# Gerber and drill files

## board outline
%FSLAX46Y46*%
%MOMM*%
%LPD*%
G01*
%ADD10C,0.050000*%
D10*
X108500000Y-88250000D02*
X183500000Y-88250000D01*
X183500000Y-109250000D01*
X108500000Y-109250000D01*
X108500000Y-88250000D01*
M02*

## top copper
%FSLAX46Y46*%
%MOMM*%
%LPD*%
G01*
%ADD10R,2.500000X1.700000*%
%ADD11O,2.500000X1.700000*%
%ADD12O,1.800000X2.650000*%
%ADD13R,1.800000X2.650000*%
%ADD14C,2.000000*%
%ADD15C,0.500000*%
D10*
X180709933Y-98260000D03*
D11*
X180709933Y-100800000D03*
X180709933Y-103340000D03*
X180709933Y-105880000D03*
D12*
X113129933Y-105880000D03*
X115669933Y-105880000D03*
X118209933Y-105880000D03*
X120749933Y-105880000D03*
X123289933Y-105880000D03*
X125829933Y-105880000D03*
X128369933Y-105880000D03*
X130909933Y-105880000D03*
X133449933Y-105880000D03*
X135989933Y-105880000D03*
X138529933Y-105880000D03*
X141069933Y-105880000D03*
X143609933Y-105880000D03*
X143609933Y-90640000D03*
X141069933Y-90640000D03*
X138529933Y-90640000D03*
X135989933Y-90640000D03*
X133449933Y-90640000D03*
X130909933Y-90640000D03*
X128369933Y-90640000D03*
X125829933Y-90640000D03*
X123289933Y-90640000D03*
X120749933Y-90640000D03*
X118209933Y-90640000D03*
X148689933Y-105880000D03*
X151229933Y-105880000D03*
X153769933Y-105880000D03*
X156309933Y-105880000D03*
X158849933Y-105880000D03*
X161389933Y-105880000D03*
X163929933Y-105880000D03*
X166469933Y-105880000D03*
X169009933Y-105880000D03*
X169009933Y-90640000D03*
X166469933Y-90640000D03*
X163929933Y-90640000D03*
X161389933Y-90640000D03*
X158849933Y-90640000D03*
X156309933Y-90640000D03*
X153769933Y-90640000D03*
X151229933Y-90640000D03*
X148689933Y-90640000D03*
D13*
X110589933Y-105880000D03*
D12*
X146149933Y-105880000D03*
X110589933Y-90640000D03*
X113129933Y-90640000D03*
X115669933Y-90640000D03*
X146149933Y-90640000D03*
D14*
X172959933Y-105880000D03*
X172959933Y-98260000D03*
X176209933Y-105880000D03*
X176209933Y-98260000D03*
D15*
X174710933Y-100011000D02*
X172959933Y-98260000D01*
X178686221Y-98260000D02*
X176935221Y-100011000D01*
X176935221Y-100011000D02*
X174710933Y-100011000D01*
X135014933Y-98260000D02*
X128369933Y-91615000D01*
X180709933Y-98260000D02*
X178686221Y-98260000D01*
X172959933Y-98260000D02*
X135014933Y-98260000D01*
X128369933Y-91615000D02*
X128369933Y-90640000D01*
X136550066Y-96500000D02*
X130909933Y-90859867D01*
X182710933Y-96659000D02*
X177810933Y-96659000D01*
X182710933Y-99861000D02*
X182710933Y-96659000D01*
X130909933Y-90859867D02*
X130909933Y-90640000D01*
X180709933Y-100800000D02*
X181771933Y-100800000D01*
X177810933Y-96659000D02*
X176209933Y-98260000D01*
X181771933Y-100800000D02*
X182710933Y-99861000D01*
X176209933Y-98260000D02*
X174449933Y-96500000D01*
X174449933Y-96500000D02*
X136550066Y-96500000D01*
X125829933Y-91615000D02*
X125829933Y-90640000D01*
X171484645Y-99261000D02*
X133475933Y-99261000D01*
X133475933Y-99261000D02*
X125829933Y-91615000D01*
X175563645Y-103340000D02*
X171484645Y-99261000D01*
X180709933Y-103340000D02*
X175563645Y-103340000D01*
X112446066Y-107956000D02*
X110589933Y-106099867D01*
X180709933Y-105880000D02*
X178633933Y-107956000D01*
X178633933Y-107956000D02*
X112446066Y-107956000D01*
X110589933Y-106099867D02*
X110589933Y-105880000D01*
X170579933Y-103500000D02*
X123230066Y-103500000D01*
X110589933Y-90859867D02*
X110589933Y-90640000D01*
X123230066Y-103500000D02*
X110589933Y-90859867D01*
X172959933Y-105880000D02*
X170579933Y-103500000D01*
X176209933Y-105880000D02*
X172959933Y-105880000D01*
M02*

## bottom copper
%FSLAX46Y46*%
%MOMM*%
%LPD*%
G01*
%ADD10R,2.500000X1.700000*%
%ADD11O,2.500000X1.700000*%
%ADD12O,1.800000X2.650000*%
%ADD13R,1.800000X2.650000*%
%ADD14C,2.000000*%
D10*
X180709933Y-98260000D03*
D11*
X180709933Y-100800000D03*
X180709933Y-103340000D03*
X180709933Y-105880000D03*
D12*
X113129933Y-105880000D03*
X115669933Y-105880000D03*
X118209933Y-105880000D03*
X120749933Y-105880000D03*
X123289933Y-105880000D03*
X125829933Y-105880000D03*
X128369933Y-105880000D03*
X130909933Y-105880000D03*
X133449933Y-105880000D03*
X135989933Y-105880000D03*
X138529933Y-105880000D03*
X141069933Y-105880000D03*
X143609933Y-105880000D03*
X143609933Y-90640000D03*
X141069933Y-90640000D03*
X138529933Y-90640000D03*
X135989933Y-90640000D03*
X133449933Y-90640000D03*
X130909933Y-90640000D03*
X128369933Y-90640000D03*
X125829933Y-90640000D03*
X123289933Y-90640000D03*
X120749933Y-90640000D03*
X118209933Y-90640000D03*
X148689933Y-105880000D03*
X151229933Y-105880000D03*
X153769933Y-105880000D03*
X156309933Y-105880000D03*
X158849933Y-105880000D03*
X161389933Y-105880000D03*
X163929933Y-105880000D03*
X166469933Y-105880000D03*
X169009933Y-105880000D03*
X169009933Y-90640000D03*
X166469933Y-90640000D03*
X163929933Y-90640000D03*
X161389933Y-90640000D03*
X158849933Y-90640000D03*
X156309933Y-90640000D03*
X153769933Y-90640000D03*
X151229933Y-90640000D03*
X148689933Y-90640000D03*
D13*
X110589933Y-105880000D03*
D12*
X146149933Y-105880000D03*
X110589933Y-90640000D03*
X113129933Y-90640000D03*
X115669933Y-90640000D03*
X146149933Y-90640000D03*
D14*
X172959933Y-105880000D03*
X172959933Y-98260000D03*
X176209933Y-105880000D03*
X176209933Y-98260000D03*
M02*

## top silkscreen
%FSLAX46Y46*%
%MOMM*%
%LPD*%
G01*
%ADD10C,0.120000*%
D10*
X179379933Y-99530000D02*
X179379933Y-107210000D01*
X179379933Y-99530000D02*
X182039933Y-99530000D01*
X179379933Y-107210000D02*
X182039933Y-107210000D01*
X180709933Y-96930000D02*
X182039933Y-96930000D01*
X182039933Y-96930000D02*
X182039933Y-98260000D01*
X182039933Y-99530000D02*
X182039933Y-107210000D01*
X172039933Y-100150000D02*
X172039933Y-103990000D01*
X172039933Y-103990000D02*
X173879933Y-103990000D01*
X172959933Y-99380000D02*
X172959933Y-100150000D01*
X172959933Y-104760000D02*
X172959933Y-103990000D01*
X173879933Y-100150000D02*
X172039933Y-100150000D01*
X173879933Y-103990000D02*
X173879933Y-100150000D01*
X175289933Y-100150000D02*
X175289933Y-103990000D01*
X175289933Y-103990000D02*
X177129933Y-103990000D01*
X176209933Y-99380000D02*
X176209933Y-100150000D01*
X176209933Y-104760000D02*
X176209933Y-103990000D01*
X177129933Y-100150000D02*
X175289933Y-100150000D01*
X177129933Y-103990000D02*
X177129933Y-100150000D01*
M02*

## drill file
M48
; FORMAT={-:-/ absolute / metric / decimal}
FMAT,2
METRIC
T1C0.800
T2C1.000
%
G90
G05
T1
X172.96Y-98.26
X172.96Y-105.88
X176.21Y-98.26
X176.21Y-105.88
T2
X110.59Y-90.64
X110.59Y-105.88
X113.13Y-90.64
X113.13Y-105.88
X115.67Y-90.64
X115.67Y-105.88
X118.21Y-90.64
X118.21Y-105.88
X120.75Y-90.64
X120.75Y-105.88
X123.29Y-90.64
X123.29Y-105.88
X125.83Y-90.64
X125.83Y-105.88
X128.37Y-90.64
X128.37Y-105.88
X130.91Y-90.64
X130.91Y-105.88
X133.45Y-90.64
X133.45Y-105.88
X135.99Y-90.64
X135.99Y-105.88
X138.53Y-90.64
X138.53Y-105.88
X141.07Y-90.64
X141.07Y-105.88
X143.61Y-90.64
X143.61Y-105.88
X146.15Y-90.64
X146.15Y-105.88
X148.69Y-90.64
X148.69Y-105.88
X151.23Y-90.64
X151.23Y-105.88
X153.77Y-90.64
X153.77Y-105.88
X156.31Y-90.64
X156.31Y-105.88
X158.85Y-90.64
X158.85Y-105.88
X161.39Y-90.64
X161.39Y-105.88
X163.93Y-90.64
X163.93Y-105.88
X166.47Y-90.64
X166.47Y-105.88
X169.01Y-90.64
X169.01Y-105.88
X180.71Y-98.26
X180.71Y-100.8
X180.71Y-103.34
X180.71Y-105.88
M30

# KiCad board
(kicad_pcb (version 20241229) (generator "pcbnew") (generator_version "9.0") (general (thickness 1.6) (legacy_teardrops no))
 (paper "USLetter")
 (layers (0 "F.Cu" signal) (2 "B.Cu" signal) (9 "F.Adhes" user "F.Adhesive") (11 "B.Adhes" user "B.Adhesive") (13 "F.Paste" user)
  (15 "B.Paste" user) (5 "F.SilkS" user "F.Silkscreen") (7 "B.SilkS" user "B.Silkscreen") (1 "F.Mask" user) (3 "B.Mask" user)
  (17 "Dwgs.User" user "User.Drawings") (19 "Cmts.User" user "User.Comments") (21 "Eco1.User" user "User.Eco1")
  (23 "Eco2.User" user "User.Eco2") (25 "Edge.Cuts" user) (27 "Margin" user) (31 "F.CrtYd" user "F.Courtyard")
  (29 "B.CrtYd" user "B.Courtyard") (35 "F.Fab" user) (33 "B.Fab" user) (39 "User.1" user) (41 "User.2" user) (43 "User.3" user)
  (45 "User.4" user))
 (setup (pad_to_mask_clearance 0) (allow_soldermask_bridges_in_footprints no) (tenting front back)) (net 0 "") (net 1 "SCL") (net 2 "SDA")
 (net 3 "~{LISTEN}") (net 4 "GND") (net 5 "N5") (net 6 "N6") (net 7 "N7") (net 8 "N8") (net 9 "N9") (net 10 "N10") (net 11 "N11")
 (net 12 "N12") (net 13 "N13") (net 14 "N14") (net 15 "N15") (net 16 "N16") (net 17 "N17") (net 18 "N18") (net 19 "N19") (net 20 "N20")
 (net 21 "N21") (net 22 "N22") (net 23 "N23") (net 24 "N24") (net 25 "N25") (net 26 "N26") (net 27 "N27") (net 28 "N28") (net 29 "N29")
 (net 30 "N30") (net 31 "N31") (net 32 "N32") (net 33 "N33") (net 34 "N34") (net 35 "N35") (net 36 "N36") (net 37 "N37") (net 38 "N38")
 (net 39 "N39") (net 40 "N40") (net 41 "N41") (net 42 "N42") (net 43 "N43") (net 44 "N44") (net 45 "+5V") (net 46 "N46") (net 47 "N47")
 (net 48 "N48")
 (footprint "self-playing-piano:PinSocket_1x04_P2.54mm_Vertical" (layer "F.Cu") (at 180.709933 98.26)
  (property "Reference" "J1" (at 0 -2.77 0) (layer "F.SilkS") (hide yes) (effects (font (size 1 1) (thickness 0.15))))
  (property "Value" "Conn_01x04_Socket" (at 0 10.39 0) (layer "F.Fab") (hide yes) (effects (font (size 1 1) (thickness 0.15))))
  (fp_line (start -1.33 1.27) (end -1.33 8.95) (stroke (width 0.12) (type solid)) (layer "F.SilkS"))
  (fp_line (start -1.33 1.27) (end 1.33 1.27) (stroke (width 0.12) (type solid)) (layer "F.SilkS"))
  (fp_line (start -1.33 8.95) (end 1.33 8.95) (stroke (width 0.12) (type solid)) (layer "F.SilkS"))
  (fp_line (start 0 -1.33) (end 1.33 -1.33) (stroke (width 0.12) (type solid)) (layer "F.SilkS"))
  (fp_line (start 1.33 -1.33) (end 1.33 0) (stroke (width 0.12) (type solid)) (layer "F.SilkS"))
  (fp_line (start 1.33 1.27) (end 1.33 8.95) (stroke (width 0.12) (type solid)) (layer "F.SilkS"))
  (pad "1" thru_hole rect (at 0 0) (size 2.5 1.7) (drill 1) (layers "*.Cu" "*.Mask") (remove_unused_layers no) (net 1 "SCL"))
  (pad "2" thru_hole oval (at 0 2.54) (size 2.5 1.7) (drill 1) (layers "*.Cu" "*.Mask") (remove_unused_layers no) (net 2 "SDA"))
  (pad "3" thru_hole oval (at 0 5.08) (size 2.5 1.7) (drill 1) (layers "*.Cu" "*.Mask") (remove_unused_layers no) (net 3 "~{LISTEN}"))
  (pad "4" thru_hole oval (at 0 7.62) (size 2.5 1.7) (drill 1) (layers "*.Cu" "*.Mask") (remove_unused_layers no) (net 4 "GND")))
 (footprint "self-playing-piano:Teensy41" (layer "F.Cu") (at 110.589933 105.88 90)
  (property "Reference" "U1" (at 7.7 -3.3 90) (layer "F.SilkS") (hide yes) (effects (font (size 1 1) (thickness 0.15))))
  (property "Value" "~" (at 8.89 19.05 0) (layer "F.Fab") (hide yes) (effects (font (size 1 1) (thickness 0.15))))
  (pad "0" thru_hole oval (at 0 2.54 90) (size 2.65 1.8) (drill 1) (layers "*.Cu" "*.Mask") (remove_unused_layers no) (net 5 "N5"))
  (pad "1" thru_hole oval (at 0 5.08 90) (size 2.65 1.8) (drill 1) (layers "*.Cu" "*.Mask") (remove_unused_layers no) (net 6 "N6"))
  (pad "2" thru_hole oval (at 0 7.62 90) (size 2.65 1.8) (drill 1) (layers "*.Cu" "*.Mask") (remove_unused_layers no) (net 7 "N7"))
  (pad "3" thru_hole oval (at 0 10.16 90) (size 2.65 1.8) (drill 1) (layers "*.Cu" "*.Mask") (remove_unused_layers no) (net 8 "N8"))
  (pad "4" thru_hole oval (at 0 12.7 90) (size 2.65 1.8) (drill 1) (layers "*.Cu" "*.Mask") (remove_unused_layers no) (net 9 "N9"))
  (pad "5" thru_hole oval (at 0 15.24 90) (size 2.65 1.8) (drill 1) (layers "*.Cu" "*.Mask") (remove_unused_layers no) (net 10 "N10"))
  (pad "6" thru_hole oval (at 0 17.78 90) (size 2.65 1.8) (drill 1) (layers "*.Cu" "*.Mask") (remove_unused_layers no) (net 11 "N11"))
  (pad "7" thru_hole oval (at 0 20.32 90) (size 2.65 1.8) (drill 1) (layers "*.Cu" "*.Mask") (remove_unused_layers no) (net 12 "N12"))
  (pad "8" thru_hole oval (at 0 22.86 90) (size 2.65 1.8) (drill 1) (layers "*.Cu" "*.Mask") (remove_unused_layers no) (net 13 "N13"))
  (pad "9" thru_hole oval (at 0 25.4 90) (size 2.65 1.8) (drill 1) (layers "*.Cu" "*.Mask") (remove_unused_layers no) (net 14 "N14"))
  (pad "10" thru_hole oval (at 0 27.94 90) (size 2.65 1.8) (drill 1) (layers "*.Cu" "*.Mask") (remove_unused_layers no) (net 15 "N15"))
  (pad "11" thru_hole oval (at 0 30.48 90) (size 2.65 1.8) (drill 1) (layers "*.Cu" "*.Mask") (remove_unused_layers no) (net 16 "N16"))
  (pad "12" thru_hole oval (at 0 33.02 90) (size 2.65 1.8) (drill 1) (layers "*.Cu" "*.Mask") (remove_unused_layers no) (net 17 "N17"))
  (pad "13" thru_hole oval (at 15.24 33.02 90) (size 2.65 1.8) (drill 1) (layers "*.Cu" "*.Mask") (remove_unused_layers no) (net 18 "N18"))
  (pad "14" thru_hole oval (at 15.24 30.48 90) (size 2.65 1.8) (drill 1) (layers "*.Cu" "*.Mask") (remove_unused_layers no) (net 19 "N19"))
  (pad "15" thru_hole oval (at 15.24 27.94 90) (size 2.65 1.8) (drill 1) (layers "*.Cu" "*.Mask") (remove_unused_layers no) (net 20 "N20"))
  (pad "16" thru_hole oval (at 15.24 25.4 90) (size 2.65 1.8) (drill 1) (layers "*.Cu" "*.Mask") (remove_unused_layers no) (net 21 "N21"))
  (pad "17" thru_hole oval (at 15.24 22.86 90) (size 2.65 1.8) (drill 1) (layers "*.Cu" "*.Mask") (remove_unused_layers no) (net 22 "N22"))
  (pad "18" thru_hole oval (at 15.24 20.32 90) (size 2.65 1.8) (drill 1) (layers "*.Cu" "*.Mask") (remove_unused_layers no) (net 2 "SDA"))
  (pad "19" thru_hole oval (at 15.24 17.78 90) (size 2.65 1.8) (drill 1) (layers "*.Cu" "*.Mask") (remove_unused_layers no) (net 1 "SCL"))
  (pad "20" thru_hole oval (at 15.24 15.24 90) (size 2.65 1.8) (drill 1) (layers "*.Cu" "*.Mask") (remove_unused_layers no)
   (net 3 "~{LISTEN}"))
  (pad "21" thru_hole oval (at 15.24 12.7 90) (size 2.65 1.8) (drill 1) (layers "*.Cu" "*.Mask") (remove_unused_layers no) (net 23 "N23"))
  (pad "22" thru_hole oval (at 15.24 10.16 90) (size 2.65 1.8) (drill 1) (layers "*.Cu" "*.Mask") (remove_unused_layers no) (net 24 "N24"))
  (pad "23" thru_hole oval (at 15.24 7.62 90) (size 2.65 1.8) (drill 1) (layers "*.Cu" "*.Mask") (remove_unused_layers no) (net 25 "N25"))
  (pad "24" thru_hole oval (at 0 38.1 90) (size 2.65 1.8) (drill 1) (layers "*.Cu" "*.Mask") (remove_unused_layers no) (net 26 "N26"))
  (pad "25" thru_hole oval (at 0 40.64 90) (size 2.65 1.8) (drill 1) (layers "*.Cu" "*.Mask") (remove_unused_layers no) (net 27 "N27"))
  (pad "26" thru_hole oval (at 0 43.18 90) (size 2.65 1.8) (drill 1) (layers "*.Cu" "*.Mask") (remove_unused_layers no) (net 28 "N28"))
  (pad "27" thru_hole oval (at 0 45.72 90) (size 2.65 1.8) (drill 1) (layers "*.Cu" "*.Mask") (remove_unused_layers no) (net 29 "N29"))
  (pad "28" thru_hole oval (at 0 48.26 90) (size 2.65 1.8) (drill 1) (layers "*.Cu" "*.Mask") (remove_unused_layers no) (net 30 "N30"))
  (pad "29" thru_hole oval (at 0 50.8 90) (size 2.65 1.8) (drill 1) (layers "*.Cu" "*.Mask") (remove_unused_layers no) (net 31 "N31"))
  (pad "30" thru_hole oval (at 0 53.34 90) (size 2.65 1.8) (drill 1) (layers "*.Cu" "*.Mask") (remove_unused_layers no) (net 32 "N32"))
  (pad "31" thru_hole oval (at 0 55.88 90) (size 2.65 1.8) (drill 1) (layers "*.Cu" "*.Mask") (remove_unused_layers no) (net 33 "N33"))
  (pad "32" thru_hole oval (at 0 58.42 90) (size 2.65 1.8) (drill 1) (layers "*.Cu" "*.Mask") (remove_unused_layers no) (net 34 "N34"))
  (pad "33" thru_hole oval (at 15.24 58.42 90) (size 2.65 1.8) (drill 1) (layers "*.Cu" "*.Mask") (remove_unused_layers no) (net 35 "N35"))
  (pad "34" thru_hole oval (at 15.24 55.88 90) (size 2.65 1.8) (drill 1) (layers "*.Cu" "*.Mask") (remove_unused_layers no) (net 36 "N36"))
  (pad "35" thru_hole oval (at 15.24 53.34 90) (size 2.65 1.8) (drill 1) (layers "*.Cu" "*.Mask") (remove_unused_layers no) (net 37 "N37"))
  (pad "36" thru_hole oval (at 15.24 50.8 90) (size 2.65 1.8) (drill 1) (layers "*.Cu" "*.Mask") (remove_unused_layers no) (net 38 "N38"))
  (pad "37" thru_hole oval (at 15.24 48.26 90) (size 2.65 1.8) (drill 1) (layers "*.Cu" "*.Mask") (remove_unused_layers no) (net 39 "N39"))
  (pad "38" thru_hole oval (at 15.24 45.72 90) (size 2.65 1.8) (drill 1) (layers "*.Cu" "*.Mask") (remove_unused_layers no) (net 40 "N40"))
  (pad "39" thru_hole oval (at 15.24 43.18 90) (size 2.65 1.8) (drill 1) (layers "*.Cu" "*.Mask") (remove_unused_layers no) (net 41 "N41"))
  (pad "40" thru_hole oval (at 15.24 40.64 90) (size 2.65 1.8) (drill 1) (layers "*.Cu" "*.Mask") (remove_unused_layers no) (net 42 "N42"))
  (pad "41" thru_hole oval (at 15.24 38.1 90) (size 2.65 1.8) (drill 1) (layers "*.Cu" "*.Mask") (remove_unused_layers no) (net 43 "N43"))
  (pad "43" thru_hole rect (at 0 0 90) (size 2.65 1.8) (drill 1) (layers "*.Cu" "*.Mask") (remove_unused_layers no) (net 4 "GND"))
  (pad "44" thru_hole oval (at 0 35.56 90) (size 2.65 1.8) (drill 1) (layers "*.Cu" "*.Mask") (remove_unused_layers no) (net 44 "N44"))
  (pad "45" thru_hole oval (at 15.24 0 90) (size 2.65 1.8) (drill 1) (layers "*.Cu" "*.Mask") (remove_unused_layers no) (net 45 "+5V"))
  (pad "46" thru_hole oval (at 15.24 2.54 90) (size 2.65 1.8) (drill 1) (layers "*.Cu" "*.Mask") (remove_unused_layers no) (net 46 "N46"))
  (pad "47" thru_hole oval (at 15.24 5.08 90) (size 2.65 1.8) (drill 1) (layers "*.Cu" "*.Mask") (remove_unused_layers no) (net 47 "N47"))
  (pad "48" thru_hole oval (at 15.24 35.56 90) (size 2.65 1.8) (drill 1) (layers "*.Cu" "*.Mask") (remove_unused_layers no) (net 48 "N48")))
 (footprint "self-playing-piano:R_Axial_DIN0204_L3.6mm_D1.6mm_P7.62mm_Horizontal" (layer "F.Cu") (at 172.959933 105.88 90)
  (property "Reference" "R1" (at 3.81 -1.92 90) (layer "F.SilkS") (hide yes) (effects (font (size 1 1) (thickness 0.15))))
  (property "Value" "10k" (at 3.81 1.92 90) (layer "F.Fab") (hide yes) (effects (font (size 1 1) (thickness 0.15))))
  (fp_line (start 5.73 -0.92) (end 1.89 -0.92) (stroke (width 0.12) (type solid)) (layer "F.SilkS"))
  (fp_line (start 1.89 -0.92) (end 1.89 0.92) (stroke (width 0.12) (type solid)) (layer "F.SilkS"))
  (fp_line (start 6.5 0) (end 5.73 0) (stroke (width 0.12) (type solid)) (layer "F.SilkS"))
  (fp_line (start 1.12 0) (end 1.89 0) (stroke (width 0.12) (type solid)) (layer "F.SilkS"))
  (fp_line (start 5.73 0.92) (end 5.73 -0.92) (stroke (width 0.12) (type solid)) (layer "F.SilkS"))
  (fp_line (start 1.89 0.92) (end 5.73 0.92) (stroke (width 0.12) (type solid)) (layer "F.SilkS"))
  (pad "1" thru_hole circle (at 0 0 90) (size 2 2) (drill 0.8) (layers "*.Cu" "*.Mask") (remove_unused_layers no) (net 45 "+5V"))
  (pad "2" thru_hole circle (at 7.62 0 90) (size 2 2) (drill 0.8) (layers "*.Cu" "*.Mask") (remove_unused_layers no) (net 1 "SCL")))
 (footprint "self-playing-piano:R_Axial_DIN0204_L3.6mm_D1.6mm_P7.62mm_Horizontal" (layer "F.Cu") (at 176.209933 105.88 90)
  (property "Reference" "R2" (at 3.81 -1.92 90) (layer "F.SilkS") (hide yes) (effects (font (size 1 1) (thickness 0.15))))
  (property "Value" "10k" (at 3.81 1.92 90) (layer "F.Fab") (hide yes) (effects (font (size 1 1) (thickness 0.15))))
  (fp_line (start 5.73 -0.92) (end 1.89 -0.92) (stroke (width 0.12) (type solid)) (layer "F.SilkS"))
  (fp_line (start 1.89 -0.92) (end 1.89 0.92) (stroke (width 0.12) (type solid)) (layer "F.SilkS"))
  (fp_line (start 6.5 0) (end 5.73 0) (stroke (width 0.12) (type solid)) (layer "F.SilkS"))
  (fp_line (start 1.12 0) (end 1.89 0) (stroke (width 0.12) (type solid)) (layer "F.SilkS"))
  (fp_line (start 5.73 0.92) (end 5.73 -0.92) (stroke (width 0.12) (type solid)) (layer "F.SilkS"))
  (fp_line (start 1.89 0.92) (end 5.73 0.92) (stroke (width 0.12) (type solid)) (layer "F.SilkS"))
  (pad "1" thru_hole circle (at 0 0 90) (size 2 2) (drill 0.8) (layers "*.Cu" "*.Mask") (remove_unused_layers no) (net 45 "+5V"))
  (pad "2" thru_hole circle (at 7.62 0 90) (size 2 2) (drill 0.8) (layers "*.Cu" "*.Mask") (remove_unused_layers no) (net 2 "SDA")))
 (gr_rect (start 108.5 88.25) (end 183.5 109.25) (stroke (width 0.05) (type default)) (fill no) (layer "Edge.Cuts"))
 (segment (start 174.710933 100.011) (end 172.959933 98.26) (width 0.5) (layer "F.Cu") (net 1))
 (segment (start 178.686221 98.26) (end 176.935221 100.011) (width 0.5) (layer "F.Cu") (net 1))
 (segment (start 176.935221 100.011) (end 174.710933 100.011) (width 0.5) (layer "F.Cu") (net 1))
 (segment (start 135.014933 98.26) (end 128.369933 91.615) (width 0.5) (layer "F.Cu") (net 1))
 (segment (start 180.709933 98.26) (end 178.686221 98.26) (width 0.5) (layer "F.Cu") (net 1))
 (segment (start 172.959933 98.26) (end 135.014933 98.26) (width 0.5) (layer "F.Cu") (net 1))
 (segment (start 128.369933 91.615) (end 128.369933 90.64) (width 0.5) (layer "F.Cu") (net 1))
 (segment (start 136.550066 96.5) (end 130.909933 90.859867) (width 0.5) (layer "F.Cu") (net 2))
 (segment (start 182.710933 96.659) (end 177.810933 96.659) (width 0.5) (layer "F.Cu") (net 2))
 (segment (start 182.710933 99.861) (end 182.710933 96.659) (width 0.5) (layer "F.Cu") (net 2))
 (segment (start 130.909933 90.859867) (end 130.909933 90.64) (width 0.5) (layer "F.Cu") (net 2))
 (segment (start 180.709933 100.8) (end 181.771933 100.8) (width 0.5) (layer "F.Cu") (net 2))
 (segment (start 177.810933 96.659) (end 176.209933 98.26) (width 0.5) (layer "F.Cu") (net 2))
 (segment (start 181.771933 100.8) (end 182.710933 99.861) (width 0.5) (layer "F.Cu") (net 2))
 (segment (start 176.209933 98.26) (end 174.449933 96.5) (width 0.5) (layer "F.Cu") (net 2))
 (segment (start 174.449933 96.5) (end 136.550066 96.5) (width 0.5) (layer "F.Cu") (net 2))
 (segment (start 125.829933 91.615) (end 125.829933 90.64) (width 0.5) (layer "F.Cu") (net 3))
 (segment (start 171.484645 99.261) (end 133.475933 99.261) (width 0.5) (layer "F.Cu") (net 3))
 (segment (start 133.475933 99.261) (end 125.829933 91.615) (width 0.5) (layer "F.Cu") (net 3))
 (segment (start 175.563645 103.34) (end 171.484645 99.261) (width 0.5) (layer "F.Cu") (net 3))
 (segment (start 180.709933 103.34) (end 175.563645 103.34) (width 0.5) (layer "F.Cu") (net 3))
 (segment (start 112.446066 107.956) (end 110.589933 106.099867) (width 0.5) (layer "F.Cu") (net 4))
 (segment (start 180.709933 105.88) (end 178.633933 107.956) (width 0.5) (layer "F.Cu") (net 4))
 (segment (start 178.633933 107.956) (end 112.446066 107.956) (width 0.5) (layer "F.Cu") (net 4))
 (segment (start 110.589933 106.099867) (end 110.589933 105.88) (width 0.5) (layer "F.Cu") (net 4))
 (segment (start 170.579933 103.5) (end 123.230066 103.5) (width 0.5) (layer "F.Cu") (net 45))
 (segment (start 110.589933 90.859867) (end 110.589933 90.64) (width 0.5) (layer "F.Cu") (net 45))
 (segment (start 123.230066 103.5) (end 110.589933 90.859867) (width 0.5) (layer "F.Cu") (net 45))
 (segment (start 172.959933 105.88) (end 170.579933 103.5) (width 0.5) (layer "F.Cu") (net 45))
 (segment (start 176.209933 105.88) (end 172.959933 105.88) (width 0.5) (layer "F.Cu") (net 45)))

